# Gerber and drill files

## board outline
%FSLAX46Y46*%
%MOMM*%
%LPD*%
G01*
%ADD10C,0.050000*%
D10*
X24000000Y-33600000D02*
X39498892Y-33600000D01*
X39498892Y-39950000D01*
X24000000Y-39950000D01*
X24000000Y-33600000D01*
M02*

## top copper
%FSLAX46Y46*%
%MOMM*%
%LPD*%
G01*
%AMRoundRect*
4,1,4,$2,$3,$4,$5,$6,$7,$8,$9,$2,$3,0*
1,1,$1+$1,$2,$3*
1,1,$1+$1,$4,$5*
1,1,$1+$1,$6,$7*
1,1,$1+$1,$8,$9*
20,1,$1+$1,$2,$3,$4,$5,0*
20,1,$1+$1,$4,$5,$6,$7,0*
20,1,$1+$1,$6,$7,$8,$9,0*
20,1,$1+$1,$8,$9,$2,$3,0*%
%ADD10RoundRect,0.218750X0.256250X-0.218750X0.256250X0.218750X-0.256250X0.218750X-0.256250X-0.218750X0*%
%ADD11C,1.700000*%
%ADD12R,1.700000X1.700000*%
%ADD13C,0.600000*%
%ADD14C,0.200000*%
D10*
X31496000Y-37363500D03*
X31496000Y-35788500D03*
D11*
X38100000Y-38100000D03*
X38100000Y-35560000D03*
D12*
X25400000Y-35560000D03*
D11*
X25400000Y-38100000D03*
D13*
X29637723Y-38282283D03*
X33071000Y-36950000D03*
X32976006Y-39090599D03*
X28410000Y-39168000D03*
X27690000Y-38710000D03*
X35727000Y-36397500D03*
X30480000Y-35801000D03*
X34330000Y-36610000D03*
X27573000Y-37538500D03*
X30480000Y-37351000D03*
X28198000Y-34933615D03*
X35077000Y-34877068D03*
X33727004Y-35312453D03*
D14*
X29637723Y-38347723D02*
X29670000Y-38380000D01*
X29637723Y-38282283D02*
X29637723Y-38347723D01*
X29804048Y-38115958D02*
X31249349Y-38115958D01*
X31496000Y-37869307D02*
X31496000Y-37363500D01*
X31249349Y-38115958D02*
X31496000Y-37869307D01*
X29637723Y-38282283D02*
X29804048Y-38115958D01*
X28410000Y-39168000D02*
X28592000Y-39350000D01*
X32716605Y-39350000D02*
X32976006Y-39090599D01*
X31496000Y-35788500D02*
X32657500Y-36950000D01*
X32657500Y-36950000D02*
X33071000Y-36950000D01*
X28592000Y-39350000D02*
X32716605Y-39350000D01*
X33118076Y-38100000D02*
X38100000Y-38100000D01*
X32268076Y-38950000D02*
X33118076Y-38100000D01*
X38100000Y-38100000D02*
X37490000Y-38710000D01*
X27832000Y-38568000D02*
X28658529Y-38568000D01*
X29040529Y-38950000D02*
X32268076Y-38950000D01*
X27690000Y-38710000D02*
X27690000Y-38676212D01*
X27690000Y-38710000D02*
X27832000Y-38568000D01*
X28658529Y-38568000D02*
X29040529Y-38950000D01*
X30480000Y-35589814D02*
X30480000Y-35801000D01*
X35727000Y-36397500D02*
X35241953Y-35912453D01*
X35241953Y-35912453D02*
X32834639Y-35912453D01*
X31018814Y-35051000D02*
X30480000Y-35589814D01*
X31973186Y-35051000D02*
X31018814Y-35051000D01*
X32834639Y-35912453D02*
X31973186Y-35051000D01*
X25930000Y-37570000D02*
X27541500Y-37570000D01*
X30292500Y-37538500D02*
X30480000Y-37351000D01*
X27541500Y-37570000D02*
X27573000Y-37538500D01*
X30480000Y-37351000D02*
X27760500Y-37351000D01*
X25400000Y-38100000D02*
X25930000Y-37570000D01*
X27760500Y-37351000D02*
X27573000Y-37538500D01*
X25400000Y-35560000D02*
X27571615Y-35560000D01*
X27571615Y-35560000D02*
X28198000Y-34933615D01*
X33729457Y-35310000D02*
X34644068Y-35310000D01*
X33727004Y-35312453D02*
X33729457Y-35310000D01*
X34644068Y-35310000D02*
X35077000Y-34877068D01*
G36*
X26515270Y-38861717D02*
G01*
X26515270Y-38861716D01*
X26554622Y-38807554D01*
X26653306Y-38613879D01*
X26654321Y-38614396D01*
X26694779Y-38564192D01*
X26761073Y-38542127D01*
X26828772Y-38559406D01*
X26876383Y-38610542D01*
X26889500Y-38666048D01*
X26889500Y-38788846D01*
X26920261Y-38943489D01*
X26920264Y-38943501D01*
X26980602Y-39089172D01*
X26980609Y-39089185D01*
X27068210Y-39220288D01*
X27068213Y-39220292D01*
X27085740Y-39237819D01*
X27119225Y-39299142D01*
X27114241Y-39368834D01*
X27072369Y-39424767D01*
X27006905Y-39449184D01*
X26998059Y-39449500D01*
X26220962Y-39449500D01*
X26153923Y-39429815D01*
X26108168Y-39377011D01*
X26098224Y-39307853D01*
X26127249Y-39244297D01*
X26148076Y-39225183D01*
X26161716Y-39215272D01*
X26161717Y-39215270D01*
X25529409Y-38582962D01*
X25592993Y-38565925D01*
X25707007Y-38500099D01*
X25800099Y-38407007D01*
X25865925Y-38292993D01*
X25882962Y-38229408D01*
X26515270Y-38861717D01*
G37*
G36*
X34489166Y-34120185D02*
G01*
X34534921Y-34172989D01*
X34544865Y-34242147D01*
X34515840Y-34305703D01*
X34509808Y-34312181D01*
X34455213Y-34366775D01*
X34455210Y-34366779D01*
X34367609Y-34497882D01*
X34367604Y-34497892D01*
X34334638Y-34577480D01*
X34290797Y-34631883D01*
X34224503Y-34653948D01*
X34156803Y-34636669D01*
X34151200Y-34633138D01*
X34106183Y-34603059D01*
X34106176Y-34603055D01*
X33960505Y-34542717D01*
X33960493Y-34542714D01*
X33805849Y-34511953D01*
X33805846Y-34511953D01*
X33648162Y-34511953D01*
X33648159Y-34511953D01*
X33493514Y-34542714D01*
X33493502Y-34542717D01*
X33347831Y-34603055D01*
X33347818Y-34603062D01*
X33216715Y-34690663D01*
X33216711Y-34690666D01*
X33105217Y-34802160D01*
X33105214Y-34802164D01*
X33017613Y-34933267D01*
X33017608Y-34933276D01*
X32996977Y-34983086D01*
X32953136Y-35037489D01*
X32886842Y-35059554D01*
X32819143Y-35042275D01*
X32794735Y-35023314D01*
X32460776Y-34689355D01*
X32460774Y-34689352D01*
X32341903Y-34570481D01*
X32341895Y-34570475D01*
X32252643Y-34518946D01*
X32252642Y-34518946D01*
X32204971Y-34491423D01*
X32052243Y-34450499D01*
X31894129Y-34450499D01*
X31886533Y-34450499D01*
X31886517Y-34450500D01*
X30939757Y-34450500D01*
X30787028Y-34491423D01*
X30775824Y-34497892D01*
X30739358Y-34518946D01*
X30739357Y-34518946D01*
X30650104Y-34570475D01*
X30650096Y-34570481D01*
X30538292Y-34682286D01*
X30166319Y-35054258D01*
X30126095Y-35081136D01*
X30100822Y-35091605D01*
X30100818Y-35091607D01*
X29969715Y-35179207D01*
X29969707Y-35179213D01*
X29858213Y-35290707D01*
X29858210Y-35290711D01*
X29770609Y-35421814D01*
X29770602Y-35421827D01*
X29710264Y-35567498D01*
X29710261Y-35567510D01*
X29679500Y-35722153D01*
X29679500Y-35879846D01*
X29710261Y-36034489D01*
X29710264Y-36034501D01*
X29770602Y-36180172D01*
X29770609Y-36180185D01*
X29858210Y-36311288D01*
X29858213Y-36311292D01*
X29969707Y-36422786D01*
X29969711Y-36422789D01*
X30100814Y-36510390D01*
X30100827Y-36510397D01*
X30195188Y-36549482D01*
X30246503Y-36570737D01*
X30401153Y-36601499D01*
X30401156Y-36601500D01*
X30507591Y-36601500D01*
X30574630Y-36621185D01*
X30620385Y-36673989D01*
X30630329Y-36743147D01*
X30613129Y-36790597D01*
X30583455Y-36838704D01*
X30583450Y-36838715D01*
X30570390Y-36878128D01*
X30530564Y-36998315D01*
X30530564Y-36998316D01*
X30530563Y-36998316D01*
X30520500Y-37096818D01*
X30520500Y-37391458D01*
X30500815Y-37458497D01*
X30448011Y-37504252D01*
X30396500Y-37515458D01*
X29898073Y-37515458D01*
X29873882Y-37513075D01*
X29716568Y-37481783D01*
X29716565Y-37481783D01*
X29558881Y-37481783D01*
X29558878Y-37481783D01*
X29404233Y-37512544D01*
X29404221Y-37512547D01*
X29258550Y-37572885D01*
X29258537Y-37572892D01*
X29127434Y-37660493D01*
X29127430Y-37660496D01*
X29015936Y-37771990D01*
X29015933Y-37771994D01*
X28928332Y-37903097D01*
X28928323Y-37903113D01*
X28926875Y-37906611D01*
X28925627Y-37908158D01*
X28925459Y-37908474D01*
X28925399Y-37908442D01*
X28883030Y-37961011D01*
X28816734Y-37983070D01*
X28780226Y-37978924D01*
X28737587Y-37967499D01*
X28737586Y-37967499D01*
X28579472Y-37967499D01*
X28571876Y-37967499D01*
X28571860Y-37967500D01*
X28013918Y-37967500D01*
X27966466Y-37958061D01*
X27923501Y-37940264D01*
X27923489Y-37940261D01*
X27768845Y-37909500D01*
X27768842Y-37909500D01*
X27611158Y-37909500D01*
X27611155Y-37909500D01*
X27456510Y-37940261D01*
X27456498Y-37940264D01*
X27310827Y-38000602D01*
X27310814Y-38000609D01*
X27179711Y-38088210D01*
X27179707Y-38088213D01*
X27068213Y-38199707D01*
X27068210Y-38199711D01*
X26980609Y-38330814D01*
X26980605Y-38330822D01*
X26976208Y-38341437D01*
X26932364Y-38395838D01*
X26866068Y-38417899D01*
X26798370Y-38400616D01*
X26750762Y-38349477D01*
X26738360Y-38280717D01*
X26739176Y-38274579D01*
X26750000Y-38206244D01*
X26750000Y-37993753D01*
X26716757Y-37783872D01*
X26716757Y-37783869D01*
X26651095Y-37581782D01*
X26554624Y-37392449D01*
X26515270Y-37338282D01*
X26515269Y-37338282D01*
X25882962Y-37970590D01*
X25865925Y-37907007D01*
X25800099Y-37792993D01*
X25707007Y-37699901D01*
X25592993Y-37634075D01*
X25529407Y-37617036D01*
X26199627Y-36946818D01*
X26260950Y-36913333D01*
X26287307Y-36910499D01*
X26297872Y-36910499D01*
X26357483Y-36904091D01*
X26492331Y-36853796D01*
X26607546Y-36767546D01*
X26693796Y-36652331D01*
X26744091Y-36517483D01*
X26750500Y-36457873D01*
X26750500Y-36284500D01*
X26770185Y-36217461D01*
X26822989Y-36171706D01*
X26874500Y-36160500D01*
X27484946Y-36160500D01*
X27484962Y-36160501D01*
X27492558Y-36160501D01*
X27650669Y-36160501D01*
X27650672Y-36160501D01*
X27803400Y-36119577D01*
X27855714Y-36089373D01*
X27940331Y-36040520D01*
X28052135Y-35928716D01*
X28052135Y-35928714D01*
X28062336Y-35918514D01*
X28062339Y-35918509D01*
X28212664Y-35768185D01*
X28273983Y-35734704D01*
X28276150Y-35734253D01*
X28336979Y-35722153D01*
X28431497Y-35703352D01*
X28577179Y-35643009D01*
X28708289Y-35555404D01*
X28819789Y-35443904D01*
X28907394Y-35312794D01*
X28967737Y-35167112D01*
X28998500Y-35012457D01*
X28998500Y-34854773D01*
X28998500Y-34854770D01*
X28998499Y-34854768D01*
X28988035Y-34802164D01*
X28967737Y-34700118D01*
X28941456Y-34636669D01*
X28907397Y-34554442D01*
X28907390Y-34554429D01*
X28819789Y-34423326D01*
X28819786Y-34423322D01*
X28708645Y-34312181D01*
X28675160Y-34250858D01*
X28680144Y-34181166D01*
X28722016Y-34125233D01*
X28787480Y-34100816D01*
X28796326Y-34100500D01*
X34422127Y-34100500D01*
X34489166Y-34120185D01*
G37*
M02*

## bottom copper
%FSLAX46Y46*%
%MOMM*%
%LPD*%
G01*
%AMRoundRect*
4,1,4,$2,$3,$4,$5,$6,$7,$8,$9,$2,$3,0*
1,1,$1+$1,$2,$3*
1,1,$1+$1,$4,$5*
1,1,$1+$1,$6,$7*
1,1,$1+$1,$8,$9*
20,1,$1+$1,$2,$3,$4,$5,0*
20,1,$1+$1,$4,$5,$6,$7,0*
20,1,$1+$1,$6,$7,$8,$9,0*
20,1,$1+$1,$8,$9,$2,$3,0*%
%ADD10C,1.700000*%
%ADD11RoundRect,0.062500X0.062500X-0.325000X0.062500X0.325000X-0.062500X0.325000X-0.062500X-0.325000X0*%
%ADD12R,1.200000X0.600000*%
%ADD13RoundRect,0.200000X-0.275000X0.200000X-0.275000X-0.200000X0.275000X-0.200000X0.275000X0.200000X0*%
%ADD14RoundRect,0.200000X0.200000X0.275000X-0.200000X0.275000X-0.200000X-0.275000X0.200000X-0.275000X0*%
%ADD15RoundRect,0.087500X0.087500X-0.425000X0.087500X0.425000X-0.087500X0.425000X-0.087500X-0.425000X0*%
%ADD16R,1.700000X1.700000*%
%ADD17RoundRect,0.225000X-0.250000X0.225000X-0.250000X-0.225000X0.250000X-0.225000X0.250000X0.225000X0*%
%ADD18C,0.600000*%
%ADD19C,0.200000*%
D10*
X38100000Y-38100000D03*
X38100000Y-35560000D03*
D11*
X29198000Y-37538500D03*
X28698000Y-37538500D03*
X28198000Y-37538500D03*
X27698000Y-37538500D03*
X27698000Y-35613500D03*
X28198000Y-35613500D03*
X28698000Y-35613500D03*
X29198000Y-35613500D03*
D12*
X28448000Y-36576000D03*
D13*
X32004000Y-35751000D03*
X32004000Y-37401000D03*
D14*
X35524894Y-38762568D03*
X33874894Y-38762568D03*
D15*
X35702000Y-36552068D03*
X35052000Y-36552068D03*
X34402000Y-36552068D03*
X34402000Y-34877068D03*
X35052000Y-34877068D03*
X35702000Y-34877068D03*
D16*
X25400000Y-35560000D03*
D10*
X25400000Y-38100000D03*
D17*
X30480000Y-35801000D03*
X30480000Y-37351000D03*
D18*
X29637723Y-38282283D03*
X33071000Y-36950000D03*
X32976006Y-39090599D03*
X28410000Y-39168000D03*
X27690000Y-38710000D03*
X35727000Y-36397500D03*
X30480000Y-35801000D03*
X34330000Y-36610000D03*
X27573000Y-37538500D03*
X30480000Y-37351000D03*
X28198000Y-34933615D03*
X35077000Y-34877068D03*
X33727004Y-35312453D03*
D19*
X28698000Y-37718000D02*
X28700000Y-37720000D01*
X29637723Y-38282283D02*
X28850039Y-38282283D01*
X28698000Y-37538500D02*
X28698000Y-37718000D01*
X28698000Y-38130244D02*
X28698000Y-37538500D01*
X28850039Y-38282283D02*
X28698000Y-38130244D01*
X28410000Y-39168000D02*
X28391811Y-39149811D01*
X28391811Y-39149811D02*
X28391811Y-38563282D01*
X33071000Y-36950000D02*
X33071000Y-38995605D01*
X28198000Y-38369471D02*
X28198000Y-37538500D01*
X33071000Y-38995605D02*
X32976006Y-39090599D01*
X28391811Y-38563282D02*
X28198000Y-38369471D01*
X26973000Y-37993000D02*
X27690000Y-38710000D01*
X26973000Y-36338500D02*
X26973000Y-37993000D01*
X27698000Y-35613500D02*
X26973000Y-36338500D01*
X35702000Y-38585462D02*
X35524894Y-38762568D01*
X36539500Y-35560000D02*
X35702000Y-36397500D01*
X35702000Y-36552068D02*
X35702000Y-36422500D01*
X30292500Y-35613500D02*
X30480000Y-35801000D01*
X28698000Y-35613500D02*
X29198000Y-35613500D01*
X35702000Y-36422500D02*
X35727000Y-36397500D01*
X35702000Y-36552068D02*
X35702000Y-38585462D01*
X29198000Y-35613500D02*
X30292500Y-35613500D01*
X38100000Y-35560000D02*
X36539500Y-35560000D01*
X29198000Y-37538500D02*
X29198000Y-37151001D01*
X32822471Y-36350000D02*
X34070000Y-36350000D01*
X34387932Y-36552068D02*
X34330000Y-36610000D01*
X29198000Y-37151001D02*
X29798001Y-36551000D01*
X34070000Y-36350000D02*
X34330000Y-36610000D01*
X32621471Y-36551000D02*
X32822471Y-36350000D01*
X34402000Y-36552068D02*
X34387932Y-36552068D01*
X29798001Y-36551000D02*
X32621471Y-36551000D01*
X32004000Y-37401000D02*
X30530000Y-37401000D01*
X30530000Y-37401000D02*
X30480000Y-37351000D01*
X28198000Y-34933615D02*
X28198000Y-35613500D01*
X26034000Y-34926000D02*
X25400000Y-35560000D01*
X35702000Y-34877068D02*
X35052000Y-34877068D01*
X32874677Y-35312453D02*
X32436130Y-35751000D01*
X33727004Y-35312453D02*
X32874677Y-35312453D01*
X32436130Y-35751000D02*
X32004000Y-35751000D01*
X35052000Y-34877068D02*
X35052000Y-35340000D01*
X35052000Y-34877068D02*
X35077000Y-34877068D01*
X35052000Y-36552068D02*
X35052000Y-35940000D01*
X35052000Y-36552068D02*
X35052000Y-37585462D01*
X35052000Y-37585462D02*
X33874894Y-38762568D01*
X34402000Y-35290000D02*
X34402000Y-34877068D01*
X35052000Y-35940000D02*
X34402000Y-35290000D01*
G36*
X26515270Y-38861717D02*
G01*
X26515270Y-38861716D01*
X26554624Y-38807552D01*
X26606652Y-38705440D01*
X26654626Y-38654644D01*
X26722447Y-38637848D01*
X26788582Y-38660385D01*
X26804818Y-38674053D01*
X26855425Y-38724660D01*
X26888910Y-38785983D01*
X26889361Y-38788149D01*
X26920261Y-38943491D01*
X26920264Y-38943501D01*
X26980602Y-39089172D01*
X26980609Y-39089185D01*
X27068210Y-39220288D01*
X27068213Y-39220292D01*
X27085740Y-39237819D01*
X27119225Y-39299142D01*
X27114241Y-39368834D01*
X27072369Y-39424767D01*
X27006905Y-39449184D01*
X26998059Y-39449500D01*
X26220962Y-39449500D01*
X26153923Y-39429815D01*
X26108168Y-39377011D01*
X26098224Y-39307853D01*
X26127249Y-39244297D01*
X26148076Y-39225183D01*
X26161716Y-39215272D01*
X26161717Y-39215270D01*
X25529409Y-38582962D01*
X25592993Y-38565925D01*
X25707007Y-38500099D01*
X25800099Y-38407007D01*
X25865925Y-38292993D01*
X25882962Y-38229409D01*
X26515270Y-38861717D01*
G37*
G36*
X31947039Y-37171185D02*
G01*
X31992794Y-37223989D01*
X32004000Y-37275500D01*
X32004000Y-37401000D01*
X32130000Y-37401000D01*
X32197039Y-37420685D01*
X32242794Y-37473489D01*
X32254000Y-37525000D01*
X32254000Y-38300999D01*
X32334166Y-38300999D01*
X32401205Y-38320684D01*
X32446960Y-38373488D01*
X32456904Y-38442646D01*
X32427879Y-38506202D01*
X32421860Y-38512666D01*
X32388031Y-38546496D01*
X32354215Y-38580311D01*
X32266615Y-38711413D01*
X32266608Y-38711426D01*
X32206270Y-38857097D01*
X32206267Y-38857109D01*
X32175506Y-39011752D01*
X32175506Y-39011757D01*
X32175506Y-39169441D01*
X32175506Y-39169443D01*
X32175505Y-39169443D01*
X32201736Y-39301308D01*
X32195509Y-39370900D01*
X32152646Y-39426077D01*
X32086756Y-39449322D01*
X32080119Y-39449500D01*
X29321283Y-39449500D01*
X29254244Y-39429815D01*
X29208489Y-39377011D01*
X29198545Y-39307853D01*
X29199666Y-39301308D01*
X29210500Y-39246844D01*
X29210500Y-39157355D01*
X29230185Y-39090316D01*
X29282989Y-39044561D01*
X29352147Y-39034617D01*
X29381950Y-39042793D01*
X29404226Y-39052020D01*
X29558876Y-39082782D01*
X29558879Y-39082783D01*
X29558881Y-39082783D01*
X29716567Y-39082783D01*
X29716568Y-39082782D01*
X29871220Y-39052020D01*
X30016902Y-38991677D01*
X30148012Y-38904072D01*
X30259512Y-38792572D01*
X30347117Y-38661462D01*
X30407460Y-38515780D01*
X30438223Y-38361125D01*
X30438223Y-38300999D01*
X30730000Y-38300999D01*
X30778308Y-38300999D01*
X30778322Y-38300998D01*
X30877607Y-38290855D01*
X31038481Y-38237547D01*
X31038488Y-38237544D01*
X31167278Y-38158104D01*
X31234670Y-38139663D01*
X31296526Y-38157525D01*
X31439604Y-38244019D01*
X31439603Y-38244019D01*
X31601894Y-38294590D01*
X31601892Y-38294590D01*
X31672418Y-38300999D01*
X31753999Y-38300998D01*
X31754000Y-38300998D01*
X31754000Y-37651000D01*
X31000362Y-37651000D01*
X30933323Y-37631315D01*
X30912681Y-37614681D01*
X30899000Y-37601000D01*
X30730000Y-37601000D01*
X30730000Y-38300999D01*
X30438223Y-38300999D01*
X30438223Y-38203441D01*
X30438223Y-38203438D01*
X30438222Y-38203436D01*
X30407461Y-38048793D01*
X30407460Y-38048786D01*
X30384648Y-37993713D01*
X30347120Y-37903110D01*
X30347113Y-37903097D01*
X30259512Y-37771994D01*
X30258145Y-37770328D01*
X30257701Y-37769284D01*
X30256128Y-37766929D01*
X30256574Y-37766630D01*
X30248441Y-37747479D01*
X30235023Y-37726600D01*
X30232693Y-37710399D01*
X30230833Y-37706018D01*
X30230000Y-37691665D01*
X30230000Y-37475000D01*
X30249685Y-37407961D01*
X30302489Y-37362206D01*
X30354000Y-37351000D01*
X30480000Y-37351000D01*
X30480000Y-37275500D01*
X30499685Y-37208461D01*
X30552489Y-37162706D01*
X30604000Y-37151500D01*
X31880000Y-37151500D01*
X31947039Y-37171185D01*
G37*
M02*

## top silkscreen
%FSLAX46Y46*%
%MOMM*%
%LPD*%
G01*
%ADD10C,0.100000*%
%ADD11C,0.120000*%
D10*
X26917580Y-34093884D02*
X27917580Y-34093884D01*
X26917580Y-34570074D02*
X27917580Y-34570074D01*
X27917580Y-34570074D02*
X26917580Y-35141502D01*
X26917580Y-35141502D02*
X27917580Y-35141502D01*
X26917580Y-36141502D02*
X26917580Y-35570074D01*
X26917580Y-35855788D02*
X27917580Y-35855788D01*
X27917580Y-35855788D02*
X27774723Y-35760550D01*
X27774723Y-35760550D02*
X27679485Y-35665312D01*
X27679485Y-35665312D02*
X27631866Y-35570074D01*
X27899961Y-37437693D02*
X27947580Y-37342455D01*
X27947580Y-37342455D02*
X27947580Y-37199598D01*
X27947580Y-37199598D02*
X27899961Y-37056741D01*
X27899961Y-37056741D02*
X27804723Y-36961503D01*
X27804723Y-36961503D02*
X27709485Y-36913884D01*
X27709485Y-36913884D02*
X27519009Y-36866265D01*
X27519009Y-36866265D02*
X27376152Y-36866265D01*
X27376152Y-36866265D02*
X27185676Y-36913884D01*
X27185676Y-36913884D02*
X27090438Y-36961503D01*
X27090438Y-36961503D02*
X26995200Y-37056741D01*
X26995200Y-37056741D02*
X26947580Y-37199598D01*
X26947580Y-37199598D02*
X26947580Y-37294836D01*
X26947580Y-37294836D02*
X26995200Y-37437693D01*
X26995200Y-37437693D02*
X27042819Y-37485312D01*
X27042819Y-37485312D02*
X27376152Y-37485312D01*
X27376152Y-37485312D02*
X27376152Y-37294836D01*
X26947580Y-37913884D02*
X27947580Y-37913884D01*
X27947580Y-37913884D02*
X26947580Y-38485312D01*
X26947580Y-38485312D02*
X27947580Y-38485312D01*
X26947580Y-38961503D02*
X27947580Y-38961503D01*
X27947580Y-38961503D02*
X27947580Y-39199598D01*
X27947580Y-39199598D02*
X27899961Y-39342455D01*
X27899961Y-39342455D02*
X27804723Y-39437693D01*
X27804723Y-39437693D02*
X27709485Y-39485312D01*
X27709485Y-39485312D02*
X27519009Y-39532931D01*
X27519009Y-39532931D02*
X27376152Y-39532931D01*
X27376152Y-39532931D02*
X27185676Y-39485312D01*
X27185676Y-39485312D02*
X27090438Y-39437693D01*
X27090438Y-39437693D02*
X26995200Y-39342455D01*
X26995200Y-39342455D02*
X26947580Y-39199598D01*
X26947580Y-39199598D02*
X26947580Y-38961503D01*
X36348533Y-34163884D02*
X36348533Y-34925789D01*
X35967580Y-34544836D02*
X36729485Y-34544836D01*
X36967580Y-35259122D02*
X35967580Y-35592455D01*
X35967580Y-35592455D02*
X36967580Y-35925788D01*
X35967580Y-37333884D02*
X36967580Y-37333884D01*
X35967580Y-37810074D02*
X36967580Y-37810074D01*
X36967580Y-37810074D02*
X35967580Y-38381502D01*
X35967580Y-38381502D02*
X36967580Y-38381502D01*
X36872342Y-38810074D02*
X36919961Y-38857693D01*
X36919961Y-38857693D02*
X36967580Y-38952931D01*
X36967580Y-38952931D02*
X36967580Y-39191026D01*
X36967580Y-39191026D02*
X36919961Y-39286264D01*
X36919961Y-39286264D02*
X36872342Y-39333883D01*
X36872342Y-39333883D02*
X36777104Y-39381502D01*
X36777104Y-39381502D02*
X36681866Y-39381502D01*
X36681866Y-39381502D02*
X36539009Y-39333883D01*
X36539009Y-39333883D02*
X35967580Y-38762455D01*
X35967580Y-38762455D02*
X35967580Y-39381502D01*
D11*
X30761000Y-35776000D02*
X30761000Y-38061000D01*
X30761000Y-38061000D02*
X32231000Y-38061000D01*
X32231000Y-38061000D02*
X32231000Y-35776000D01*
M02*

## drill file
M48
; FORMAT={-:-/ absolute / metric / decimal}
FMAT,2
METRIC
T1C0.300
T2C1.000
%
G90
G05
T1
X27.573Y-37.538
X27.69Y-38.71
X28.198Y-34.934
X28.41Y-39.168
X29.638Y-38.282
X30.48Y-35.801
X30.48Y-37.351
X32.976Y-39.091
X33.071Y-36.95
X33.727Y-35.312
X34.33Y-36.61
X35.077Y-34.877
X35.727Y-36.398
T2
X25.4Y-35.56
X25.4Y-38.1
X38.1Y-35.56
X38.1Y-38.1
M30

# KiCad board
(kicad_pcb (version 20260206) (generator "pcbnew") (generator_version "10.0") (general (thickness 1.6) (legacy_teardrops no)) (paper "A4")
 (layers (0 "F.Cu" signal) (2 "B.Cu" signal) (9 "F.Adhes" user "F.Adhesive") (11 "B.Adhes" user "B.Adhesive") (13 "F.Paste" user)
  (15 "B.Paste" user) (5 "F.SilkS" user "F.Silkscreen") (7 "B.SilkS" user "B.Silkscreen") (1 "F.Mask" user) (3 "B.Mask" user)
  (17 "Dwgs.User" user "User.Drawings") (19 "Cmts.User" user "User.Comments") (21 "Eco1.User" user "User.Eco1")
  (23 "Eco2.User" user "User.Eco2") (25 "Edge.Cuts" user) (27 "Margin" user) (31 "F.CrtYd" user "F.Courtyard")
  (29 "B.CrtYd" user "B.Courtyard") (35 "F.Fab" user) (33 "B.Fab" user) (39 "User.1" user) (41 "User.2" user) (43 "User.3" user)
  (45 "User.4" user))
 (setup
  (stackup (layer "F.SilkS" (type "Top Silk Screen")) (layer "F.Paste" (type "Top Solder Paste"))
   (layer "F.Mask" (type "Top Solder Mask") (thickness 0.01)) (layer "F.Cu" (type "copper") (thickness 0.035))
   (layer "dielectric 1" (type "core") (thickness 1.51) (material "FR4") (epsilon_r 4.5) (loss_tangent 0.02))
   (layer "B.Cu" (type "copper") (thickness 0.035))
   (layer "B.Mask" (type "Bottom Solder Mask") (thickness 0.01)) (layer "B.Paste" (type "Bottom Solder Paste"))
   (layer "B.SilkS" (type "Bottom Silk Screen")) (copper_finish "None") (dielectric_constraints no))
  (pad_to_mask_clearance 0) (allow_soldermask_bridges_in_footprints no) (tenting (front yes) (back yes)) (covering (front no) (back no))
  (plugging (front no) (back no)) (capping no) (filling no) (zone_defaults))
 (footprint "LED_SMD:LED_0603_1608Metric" (layer "F.Cu") (at 31.496 36.576 90)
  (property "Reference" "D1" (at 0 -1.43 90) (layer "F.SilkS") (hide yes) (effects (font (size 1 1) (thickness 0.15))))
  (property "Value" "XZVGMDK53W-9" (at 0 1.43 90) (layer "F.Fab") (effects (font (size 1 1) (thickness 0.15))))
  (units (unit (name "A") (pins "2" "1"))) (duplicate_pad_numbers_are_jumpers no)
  (fp_line (start 0.8 -0.735) (end -1.485 -0.735) (stroke (width 0.12) (type solid)) (layer "F.SilkS"))
  (fp_line (start -1.485 -0.735) (end -1.485 0.735) (stroke (width 0.12) (type solid)) (layer "F.SilkS"))
  (fp_line (start -1.485 0.735) (end 0.8 0.735) (stroke (width 0.12) (type solid)) (layer "F.SilkS"))
  (pad "1" smd roundrect (at -0.7875 0 90) (size 0.875 0.95) (layers "F.Cu" "F.Mask" "F.Paste") (roundrect_rratio 0.25) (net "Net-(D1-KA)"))
  (pad "2" smd roundrect (at 0.7875 0 90) (size 0.875 0.95) (layers "F.Cu" "F.Mask" "F.Paste") (roundrect_rratio 0.25) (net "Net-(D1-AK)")))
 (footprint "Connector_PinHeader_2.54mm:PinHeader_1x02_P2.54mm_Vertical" (layer "B.Cu") (at 38.1 38.1)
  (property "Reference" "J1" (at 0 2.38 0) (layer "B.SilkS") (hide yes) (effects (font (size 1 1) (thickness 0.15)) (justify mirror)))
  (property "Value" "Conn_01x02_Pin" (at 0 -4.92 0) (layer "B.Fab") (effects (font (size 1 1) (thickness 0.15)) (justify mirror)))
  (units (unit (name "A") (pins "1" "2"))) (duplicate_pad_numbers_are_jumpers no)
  (pad "1" thru_hole circle (at 0 0) (size 1.7 1.7) (drill 1) (layers "*.Cu" "*.Mask") (remove_unused_layers no) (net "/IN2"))
  (pad "2" thru_hole circle (at 0 -2.54) (size 1.7 1.7) (drill 1) (layers "*.Cu" "*.Mask") (remove_unused_layers no) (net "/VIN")))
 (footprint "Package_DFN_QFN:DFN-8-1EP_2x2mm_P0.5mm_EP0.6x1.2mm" (layer "B.Cu") (at 28.448 36.576 90)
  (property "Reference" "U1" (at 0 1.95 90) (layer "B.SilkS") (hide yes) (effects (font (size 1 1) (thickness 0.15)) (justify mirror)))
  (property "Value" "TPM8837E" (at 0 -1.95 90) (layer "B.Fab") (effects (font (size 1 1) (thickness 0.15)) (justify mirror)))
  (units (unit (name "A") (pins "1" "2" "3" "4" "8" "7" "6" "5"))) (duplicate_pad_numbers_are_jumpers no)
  (pad "" smd roundrect (at -0.15 -0.3 90) (size 0.24 0.48) (layers "B.Paste") (roundrect_rratio 0.25))
  (pad "" smd roundrect (at -0.15 0.3 90) (size 0.24 0.48) (layers "B.Paste") (roundrect_rratio 0.25))
  (pad "" smd roundrect (at 0.15 -0.3 90) (size 0.24 0.48) (layers "B.Paste") (roundrect_rratio 0.25))
  (pad "" smd roundrect (at 0.15 0.3 90) (size 0.24 0.48) (layers "B.Paste") (roundrect_rratio 0.25))
  (pad "1" smd roundrect (at -0.9625 0.75 90) (size 0.775 0.25) (layers "B.Cu" "B.Mask" "B.Paste") (roundrect_rratio 0.25)
   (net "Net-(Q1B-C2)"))
  (pad "2" smd roundrect (at -0.9625 0.25 90) (size 0.775 0.25) (layers "B.Cu" "B.Mask" "B.Paste") (roundrect_rratio 0.25)
   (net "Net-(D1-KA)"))
  (pad "3" smd roundrect (at -0.9625 -0.25 90) (size 0.775 0.25) (layers "B.Cu" "B.Mask" "B.Paste") (roundrect_rratio 0.25)
   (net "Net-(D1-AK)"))
  (pad "4" smd roundrect (at -0.9625 -0.75 90) (size 0.775 0.25) (layers "B.Cu" "B.Mask" "B.Paste") (roundrect_rratio 0.25) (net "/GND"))
  (pad "5" smd roundrect (at 0.9625 -0.75 90) (size 0.775 0.25) (layers "B.Cu" "B.Mask" "B.Paste") (roundrect_rratio 0.25) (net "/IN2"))
  (pad "6" smd roundrect (at 0.9625 -0.25 90) (size 0.775 0.25) (layers "B.Cu" "B.Mask" "B.Paste") (roundrect_rratio 0.25) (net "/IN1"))
  (pad "7" smd roundrect (at 0.9625 0.25 90) (size 0.775 0.25) (layers "B.Cu" "B.Mask" "B.Paste") (roundrect_rratio 0.25) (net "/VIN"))
  (pad "8" smd roundrect (at 0.9625 0.75 90) (size 0.775 0.25) (layers "B.Cu" "B.Mask" "B.Paste") (roundrect_rratio 0.25) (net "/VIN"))
  (pad "9" smd rect (at 0 0 90) (size 0.6 1.2) (layers "B.Cu" "B.Mask") (zone_connect 2)))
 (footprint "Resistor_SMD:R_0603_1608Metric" (layer "B.Cu") (at 32.004 36.576 -90)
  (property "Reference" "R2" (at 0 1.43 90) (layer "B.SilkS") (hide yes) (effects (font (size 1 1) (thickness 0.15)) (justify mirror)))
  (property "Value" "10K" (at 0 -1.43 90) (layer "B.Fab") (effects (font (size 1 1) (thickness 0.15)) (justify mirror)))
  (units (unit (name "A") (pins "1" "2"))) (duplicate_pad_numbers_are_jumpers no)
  (pad "1" smd roundrect (at -0.825 0 270) (size 0.8 0.95) (layers "B.Cu" "B.Mask" "B.Paste") (roundrect_rratio 0.25) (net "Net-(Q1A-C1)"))
  (pad "2" smd roundrect (at 0.825 0 270) (size 0.8 0.95) (layers "B.Cu" "B.Mask" "B.Paste") (roundrect_rratio 0.25) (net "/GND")))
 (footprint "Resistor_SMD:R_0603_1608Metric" (layer "B.Cu") (at 34.699894 38.762568 180)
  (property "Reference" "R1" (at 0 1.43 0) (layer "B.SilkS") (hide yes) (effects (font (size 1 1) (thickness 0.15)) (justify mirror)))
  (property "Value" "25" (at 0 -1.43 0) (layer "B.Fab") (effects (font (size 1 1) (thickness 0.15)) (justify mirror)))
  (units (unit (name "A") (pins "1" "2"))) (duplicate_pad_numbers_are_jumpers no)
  (pad "1" smd roundrect (at -0.825 0 180) (size 0.8 0.95) (layers "B.Cu" "B.Mask" "B.Paste") (roundrect_rratio 0.25) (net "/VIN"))
  (pad "2" smd roundrect (at 0.825 0 180) (size 0.8 0.95) (layers "B.Cu" "B.Mask" "B.Paste") (roundrect_rratio 0.25) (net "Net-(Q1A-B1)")))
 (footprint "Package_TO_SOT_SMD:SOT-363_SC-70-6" (layer "B.Cu") (at 35.052 35.714568 90)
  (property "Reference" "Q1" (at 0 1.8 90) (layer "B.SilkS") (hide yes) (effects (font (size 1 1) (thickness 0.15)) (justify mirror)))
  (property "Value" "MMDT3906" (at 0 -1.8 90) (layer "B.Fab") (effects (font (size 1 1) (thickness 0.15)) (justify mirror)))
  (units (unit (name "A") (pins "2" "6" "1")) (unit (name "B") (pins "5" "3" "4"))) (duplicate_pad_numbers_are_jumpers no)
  (pad "1" smd roundrect (at -0.8375 0.65 90) (size 1.025 0.35) (layers "B.Cu" "B.Mask" "B.Paste") (roundrect_rratio 0.25) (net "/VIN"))
  (pad "2" smd roundrect (at -0.8375 0 90) (size 1.025 0.35) (layers "B.Cu" "B.Mask" "B.Paste") (roundrect_rratio 0.25) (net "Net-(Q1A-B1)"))
  (pad "3" smd roundrect (at -0.8375 -0.65 90) (size 1.025 0.35) (layers "B.Cu" "B.Mask" "B.Paste") (roundrect_rratio 0.25)
   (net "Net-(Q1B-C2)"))
  (pad "4" smd roundrect (at 0.8375 -0.65 90) (size 1.025 0.35) (layers "B.Cu" "B.Mask" "B.Paste") (roundrect_rratio 0.25)
   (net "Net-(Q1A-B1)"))
  (pad "5" smd roundrect (at 0.8375 0 90) (size 1.025 0.35) (layers "B.Cu" "B.Mask" "B.Paste") (roundrect_rratio 0.25) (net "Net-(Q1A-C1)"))
  (pad "6" smd roundrect (at 0.8375 0.65 90) (size 1.025 0.35) (layers "B.Cu" "B.Mask" "B.Paste") (roundrect_rratio 0.25)
   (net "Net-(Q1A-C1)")))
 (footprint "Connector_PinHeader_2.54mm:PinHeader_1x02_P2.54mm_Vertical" (layer "B.Cu") (at 25.4 35.56 180)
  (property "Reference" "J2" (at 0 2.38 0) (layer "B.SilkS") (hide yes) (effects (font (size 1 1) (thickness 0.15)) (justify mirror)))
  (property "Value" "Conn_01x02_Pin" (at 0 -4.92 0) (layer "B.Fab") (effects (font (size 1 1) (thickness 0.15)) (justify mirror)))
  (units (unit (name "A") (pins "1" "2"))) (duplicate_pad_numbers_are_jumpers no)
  (pad "1" thru_hole rect (at 0 0 180) (size 1.7 1.7) (drill 1) (layers "*.Cu" "*.Mask") (remove_unused_layers no) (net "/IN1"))
  (pad "2" thru_hole circle (at 0 -2.54 180) (size 1.7 1.7) (drill 1) (layers "*.Cu" "*.Mask") (remove_unused_layers no) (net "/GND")))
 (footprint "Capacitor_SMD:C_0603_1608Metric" (layer "B.Cu") (at 30.48 36.576 -90)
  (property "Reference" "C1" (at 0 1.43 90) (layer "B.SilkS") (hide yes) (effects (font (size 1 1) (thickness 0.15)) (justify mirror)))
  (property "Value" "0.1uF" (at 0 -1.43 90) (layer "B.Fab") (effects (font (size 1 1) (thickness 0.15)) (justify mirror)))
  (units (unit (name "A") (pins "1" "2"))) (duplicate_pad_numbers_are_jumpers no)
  (pad "1" smd roundrect (at -0.775 0 270) (size 0.9 0.95) (layers "B.Cu" "B.Mask" "B.Paste") (roundrect_rratio 0.25) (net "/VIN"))
  (pad "2" smd roundrect (at 0.775 0 270) (size 0.9 0.95) (layers "B.Cu" "B.Mask" "B.Paste") (roundrect_rratio 0.25) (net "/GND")))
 (gr_rect (start 24 33.6) (end 39.498892 39.95) (stroke (width 0.05) (type solid)) (fill no) (layer "Edge.Cuts"))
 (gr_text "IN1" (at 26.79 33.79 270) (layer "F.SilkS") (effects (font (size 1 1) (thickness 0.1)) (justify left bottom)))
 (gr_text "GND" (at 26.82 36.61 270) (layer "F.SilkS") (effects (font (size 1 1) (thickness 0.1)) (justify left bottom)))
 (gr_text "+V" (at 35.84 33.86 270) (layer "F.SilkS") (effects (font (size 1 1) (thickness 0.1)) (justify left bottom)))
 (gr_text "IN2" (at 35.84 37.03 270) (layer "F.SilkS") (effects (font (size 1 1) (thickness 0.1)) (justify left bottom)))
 (segment (start 29.637723 38.347723) (end 29.67 38.38) (width 0.2) (layer "F.Cu") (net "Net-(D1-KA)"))
 (segment (start 29.637723 38.282283) (end 29.637723 38.347723) (width 0.2) (layer "F.Cu") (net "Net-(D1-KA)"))
 (segment (start 29.804048 38.115958) (end 31.249349 38.115958) (width 0.2) (layer "F.Cu") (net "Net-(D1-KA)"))
 (segment (start 31.496 37.869307) (end 31.496 37.3635) (width 0.2) (layer "F.Cu") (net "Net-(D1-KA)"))
 (segment (start 31.249349 38.115958) (end 31.496 37.869307) (width 0.2) (layer "F.Cu") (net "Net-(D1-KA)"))
 (segment (start 29.637723 38.282283) (end 29.804048 38.115958) (width 0.2) (layer "F.Cu") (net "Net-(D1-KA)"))
 (via (at 29.637723 38.282283) (size 0.6) (drill 0.3) (layers "F.Cu" "B.Cu") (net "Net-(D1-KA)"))
 (segment (start 28.698 37.718) (end 28.7 37.72) (width 0.2) (layer "B.Cu") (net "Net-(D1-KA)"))
 (segment (start 29.637723 38.282283) (end 28.850039 38.282283) (width 0.2) (layer "B.Cu") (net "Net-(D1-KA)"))
 (segment (start 28.698 37.5385) (end 28.698 37.718) (width 0.2) (layer "B.Cu") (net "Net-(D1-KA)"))
 (segment (start 28.698 38.130244) (end 28.698 37.5385) (width 0.2) (layer "B.Cu") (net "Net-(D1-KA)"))
 (segment (start 28.850039 38.282283) (end 28.698 38.130244) (width 0.2) (layer "B.Cu") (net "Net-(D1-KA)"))
 (segment (start 28.41 39.168) (end 28.592 39.35) (width 0.2) (layer "F.Cu") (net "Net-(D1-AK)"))
 (segment (start 32.716605 39.35) (end 32.976006 39.090599) (width 0.2) (layer "F.Cu") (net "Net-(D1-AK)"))
 (segment (start 31.496 35.7885) (end 32.6575 36.95) (width 0.2) (layer "F.Cu") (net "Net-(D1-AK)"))
 (segment (start 32.6575 36.95) (end 33.071 36.95) (width 0.2) (layer "F.Cu") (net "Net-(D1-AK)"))
 (segment (start 28.592 39.35) (end 32.716605 39.35) (width 0.2) (layer "F.Cu") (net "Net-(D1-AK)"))
 (via (at 33.071 36.95) (size 0.6) (drill 0.3) (layers "F.Cu" "B.Cu") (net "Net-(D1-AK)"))
 (via (at 32.976006 39.090599) (size 0.6) (drill 0.3) (layers "F.Cu" "B.Cu") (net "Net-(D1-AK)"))
 (via (at 28.41 39.168) (size 0.6) (drill 0.3) (layers "F.Cu" "B.Cu") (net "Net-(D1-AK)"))
 (segment (start 28.41 39.168) (end 28.391811 39.149811) (width 0.2) (layer "B.Cu") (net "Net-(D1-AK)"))
 (segment (start 28.391811 39.149811) (end 28.391811 38.563282) (width 0.2) (layer "B.Cu") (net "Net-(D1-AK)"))
 (segment (start 33.071 36.95) (end 33.071 38.995605) (width 0.2) (layer "B.Cu") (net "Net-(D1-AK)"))
 (segment (start 28.198 38.369471) (end 28.198 37.5385) (width 0.2) (layer "B.Cu") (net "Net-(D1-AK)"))
 (segment (start 33.071 38.995605) (end 32.976006 39.090599) (width 0.2) (layer "B.Cu") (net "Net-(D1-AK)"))
 (segment (start 28.391811 38.563282) (end 28.198 38.369471) (width 0.2) (layer "B.Cu") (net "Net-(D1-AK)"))
 (segment (start 33.118076 38.1) (end 38.1 38.1) (width 0.2) (layer "F.Cu") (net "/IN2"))
 (segment (start 32.268076 38.95) (end 33.118076 38.1) (width 0.2) (layer "F.Cu") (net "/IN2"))
 (segment (start 38.1 38.1) (end 37.49 38.71) (width 0.2) (layer "F.Cu") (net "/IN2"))
 (segment (start 27.832 38.568) (end 28.658529 38.568) (width 0.2) (layer "F.Cu") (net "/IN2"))
 (segment (start 29.040529 38.95) (end 32.268076 38.95) (width 0.2) (layer "F.Cu") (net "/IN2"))
 (segment (start 27.69 38.71) (end 27.69 38.676212) (width 0.2) (layer "F.Cu") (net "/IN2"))
 (segment (start 27.69 38.71) (end 27.832 38.568) (width 0.2) (layer "F.Cu") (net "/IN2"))
 (segment (start 28.658529 38.568) (end 29.040529 38.95) (width 0.2) (layer "F.Cu") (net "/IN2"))
 (via (at 27.69 38.71) (size 0.6) (drill 0.3) (layers "F.Cu" "B.Cu") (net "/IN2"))
 (segment (start 26.973 37.993) (end 27.69 38.71) (width 0.2) (layer "B.Cu") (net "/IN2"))
 (segment (start 26.973 36.3385) (end 26.973 37.993) (width 0.2) (layer "B.Cu") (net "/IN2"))
 (segment (start 27.698 35.6135) (end 26.973 36.3385) (width 0.2) (layer "B.Cu") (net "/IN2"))
 (segment (start 30.48 35.589814) (end 30.48 35.801) (width 0.2) (layer "F.Cu") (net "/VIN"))
 (segment (start 35.727 36.3975) (end 35.241953 35.912453) (width 0.2) (layer "F.Cu") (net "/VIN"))
 (segment (start 35.241953 35.912453) (end 32.834639 35.912453) (width 0.2) (layer "F.Cu") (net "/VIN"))
 (segment (start 31.018814 35.051) (end 30.48 35.589814) (width 0.2) (layer "F.Cu") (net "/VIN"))
 (segment (start 31.973186 35.051) (end 31.018814 35.051) (width 0.2) (layer "F.Cu") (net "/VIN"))
 (segment (start 32.834639 35.912453) (end 31.973186 35.051) (width 0.2) (layer "F.Cu") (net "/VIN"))
 (via (at 35.727 36.3975) (size 0.6) (drill 0.3) (layers "F.Cu" "B.Cu") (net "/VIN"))
 (via (at 30.48 35.801) (size 0.6) (drill 0.3) (layers "F.Cu" "B.Cu") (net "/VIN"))
 (segment (start 35.702 38.585462) (end 35.524894 38.762568) (width 0.2) (layer "B.Cu") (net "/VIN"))
 (segment (start 36.5395 35.56) (end 35.702 36.3975) (width 0.2) (layer "B.Cu") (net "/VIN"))
 (segment (start 35.702 36.552068) (end 35.702 36.4225) (width 0.2) (layer "B.Cu") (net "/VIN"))
 (segment (start 30.2925 35.6135) (end 30.48 35.801) (width 0.2) (layer "B.Cu") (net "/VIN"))
 (segment (start 28.698 35.6135) (end 29.198 35.6135) (width 0.2) (layer "B.Cu") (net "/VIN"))
 (segment (start 35.702 36.4225) (end 35.727 36.3975) (width 0.2) (layer "B.Cu") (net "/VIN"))
 (segment (start 35.702 36.552068) (end 35.702 38.585462) (width 0.2) (layer "B.Cu") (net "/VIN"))
 (segment (start 29.198 35.6135) (end 30.2925 35.6135) (width 0.2) (layer "B.Cu") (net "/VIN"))
 (segment (start 38.1 35.56) (end 36.5395 35.56) (width 0.2) (layer "B.Cu") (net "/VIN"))
 (via (at 34.33 36.61) (size 0.6) (drill 0.3) (layers "F.Cu" "B.Cu") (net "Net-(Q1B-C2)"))
 (segment (start 29.198 37.5385) (end 29.198 37.151001) (width 0.2) (layer "B.Cu") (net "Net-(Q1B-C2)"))
 (segment (start 32.822471 36.35) (end 34.07 36.35) (width 0.2) (layer "B.Cu") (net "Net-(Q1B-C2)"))
 (segment (start 34.387932 36.552068) (end 34.33 36.61) (width 0.2) (layer "B.Cu") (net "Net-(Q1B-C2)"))
 (segment (start 29.198 37.151001) (end 29.798001 36.551) (width 0.2) (layer "B.Cu") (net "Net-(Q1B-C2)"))
 (segment (start 34.07 36.35) (end 34.33 36.61) (width 0.2) (layer "B.Cu") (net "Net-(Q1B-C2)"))
 (segment (start 32.621471 36.551) (end 32.822471 36.35) (width 0.2) (layer "B.Cu") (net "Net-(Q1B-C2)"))
 (segment (start 34.402 36.552068) (end 34.387932 36.552068) (width 0.2) (layer "B.Cu") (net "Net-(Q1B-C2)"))
 (segment (start 29.798001 36.551) (end 32.621471 36.551) (width 0.2) (layer "B.Cu") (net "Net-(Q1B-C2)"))
 (segment (start 25.93 37.57) (end 27.5415 37.57) (width 0.2) (layer "F.Cu") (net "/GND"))
 (segment (start 30.2925 37.5385) (end 30.48 37.351) (width 0.2) (layer "F.Cu") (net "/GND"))
 (segment (start 27.5415 37.57) (end 27.573 37.5385) (width 0.2) (layer "F.Cu") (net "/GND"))
 (segment (start 30.48 37.351) (end 27.7605 37.351) (width 0.2) (layer "F.Cu") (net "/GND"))
 (segment (start 25.4 38.1) (end 25.93 37.57) (width 0.2) (layer "F.Cu") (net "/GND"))
 (segment (start 27.7605 37.351) (end 27.573 37.5385) (width 0.2) (layer "F.Cu") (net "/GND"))
 (via (at 27.573 37.5385) (size 0.6) (drill 0.3) (layers "F.Cu" "B.Cu") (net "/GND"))
 (via (at 30.48 37.351) (size 0.6) (drill 0.3) (layers "F.Cu" "B.Cu") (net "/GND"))
 (segment (start 32.004 37.401) (end 30.53 37.401) (width 0.2) (layer "B.Cu") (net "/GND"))
 (segment (start 30.53 37.401) (end 30.48 37.351) (width 0.2) (layer "B.Cu") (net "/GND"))
 (segment (start 25.4 35.56) (end 27.571615 35.56) (width 0.2) (layer "F.Cu") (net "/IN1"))
 (segment (start 27.571615 35.56) (end 28.198 34.933615) (width 0.2) (layer "F.Cu") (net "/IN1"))
 (via (at 28.198 34.933615) (size 0.6) (drill 0.3) (layers "F.Cu" "B.Cu") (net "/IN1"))
 (segment (start 28.198 34.933615) (end 28.198 35.6135) (width 0.2) (layer "B.Cu") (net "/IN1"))
 (segment (start 26.034 34.926) (end 25.4 35.56) (width 0.2) (layer "B.Cu") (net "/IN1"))
 (segment (start 33.729457 35.31) (end 34.644068 35.31) (width 0.2) (layer "F.Cu") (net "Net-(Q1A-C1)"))
 (segment (start 33.727004 35.312453) (end 33.729457 35.31) (width 0.2) (layer "F.Cu") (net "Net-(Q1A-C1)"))
 (segment (start 34.644068 35.31) (end 35.077 34.877068) (width 0.2) (layer "F.Cu") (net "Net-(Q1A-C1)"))
 (via (at 35.077 34.877068) (size 0.6) (drill 0.3) (layers "F.Cu" "B.Cu") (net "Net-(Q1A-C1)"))
 (via (at 33.727004 35.312453) (size 0.6) (drill 0.3) (layers "F.Cu" "B.Cu") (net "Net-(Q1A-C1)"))
 (segment (start 35.702 34.877068) (end 35.052 34.877068) (width 0.2) (layer "B.Cu") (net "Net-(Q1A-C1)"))
 (segment (start 32.874677 35.312453) (end 32.43613 35.751) (width 0.2) (layer "B.Cu") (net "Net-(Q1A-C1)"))
 (segment (start 33.727004 35.312453) (end 32.874677 35.312453) (width 0.2) (layer "B.Cu") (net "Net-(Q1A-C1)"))
 (segment (start 32.43613 35.751) (end 32.004 35.751) (width 0.2) (layer "B.Cu") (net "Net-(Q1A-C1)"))
 (segment (start 35.052 34.877068) (end 35.052 35.34) (width 0.2) (layer "B.Cu") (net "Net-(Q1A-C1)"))
 (segment (start 35.052 34.877068) (end 35.077 34.877068) (width 0.2) (layer "B.Cu") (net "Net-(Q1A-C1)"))
 (segment (start 35.052 36.552068) (end 35.052 35.94) (width 0.2) (layer "B.Cu") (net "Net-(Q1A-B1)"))
 (segment (start 35.052 36.552068) (end 35.052 37.585462) (width 0.2) (layer "B.Cu") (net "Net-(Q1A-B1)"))
 (segment (start 35.052 37.585462) (end 33.874894 38.762568) (width 0.2) (layer "B.Cu") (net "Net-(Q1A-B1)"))
 (segment (start 34.402 35.29) (end 34.402 34.877068) (width 0.2) (layer "B.Cu") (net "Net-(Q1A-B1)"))
 (segment (start 35.052 35.94) (end 34.402 35.29) (width 0.2) (layer "B.Cu") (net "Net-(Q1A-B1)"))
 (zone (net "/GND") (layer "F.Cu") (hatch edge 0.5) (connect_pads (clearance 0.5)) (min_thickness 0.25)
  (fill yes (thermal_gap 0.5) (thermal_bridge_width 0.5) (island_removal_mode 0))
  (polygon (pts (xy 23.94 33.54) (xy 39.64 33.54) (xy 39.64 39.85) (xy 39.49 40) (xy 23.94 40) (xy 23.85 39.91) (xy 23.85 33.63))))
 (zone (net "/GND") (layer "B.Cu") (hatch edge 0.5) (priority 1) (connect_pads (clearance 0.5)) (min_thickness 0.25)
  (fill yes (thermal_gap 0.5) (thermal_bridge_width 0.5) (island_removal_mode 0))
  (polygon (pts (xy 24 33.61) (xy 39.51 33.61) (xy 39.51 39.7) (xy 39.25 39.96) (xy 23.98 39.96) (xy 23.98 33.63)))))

